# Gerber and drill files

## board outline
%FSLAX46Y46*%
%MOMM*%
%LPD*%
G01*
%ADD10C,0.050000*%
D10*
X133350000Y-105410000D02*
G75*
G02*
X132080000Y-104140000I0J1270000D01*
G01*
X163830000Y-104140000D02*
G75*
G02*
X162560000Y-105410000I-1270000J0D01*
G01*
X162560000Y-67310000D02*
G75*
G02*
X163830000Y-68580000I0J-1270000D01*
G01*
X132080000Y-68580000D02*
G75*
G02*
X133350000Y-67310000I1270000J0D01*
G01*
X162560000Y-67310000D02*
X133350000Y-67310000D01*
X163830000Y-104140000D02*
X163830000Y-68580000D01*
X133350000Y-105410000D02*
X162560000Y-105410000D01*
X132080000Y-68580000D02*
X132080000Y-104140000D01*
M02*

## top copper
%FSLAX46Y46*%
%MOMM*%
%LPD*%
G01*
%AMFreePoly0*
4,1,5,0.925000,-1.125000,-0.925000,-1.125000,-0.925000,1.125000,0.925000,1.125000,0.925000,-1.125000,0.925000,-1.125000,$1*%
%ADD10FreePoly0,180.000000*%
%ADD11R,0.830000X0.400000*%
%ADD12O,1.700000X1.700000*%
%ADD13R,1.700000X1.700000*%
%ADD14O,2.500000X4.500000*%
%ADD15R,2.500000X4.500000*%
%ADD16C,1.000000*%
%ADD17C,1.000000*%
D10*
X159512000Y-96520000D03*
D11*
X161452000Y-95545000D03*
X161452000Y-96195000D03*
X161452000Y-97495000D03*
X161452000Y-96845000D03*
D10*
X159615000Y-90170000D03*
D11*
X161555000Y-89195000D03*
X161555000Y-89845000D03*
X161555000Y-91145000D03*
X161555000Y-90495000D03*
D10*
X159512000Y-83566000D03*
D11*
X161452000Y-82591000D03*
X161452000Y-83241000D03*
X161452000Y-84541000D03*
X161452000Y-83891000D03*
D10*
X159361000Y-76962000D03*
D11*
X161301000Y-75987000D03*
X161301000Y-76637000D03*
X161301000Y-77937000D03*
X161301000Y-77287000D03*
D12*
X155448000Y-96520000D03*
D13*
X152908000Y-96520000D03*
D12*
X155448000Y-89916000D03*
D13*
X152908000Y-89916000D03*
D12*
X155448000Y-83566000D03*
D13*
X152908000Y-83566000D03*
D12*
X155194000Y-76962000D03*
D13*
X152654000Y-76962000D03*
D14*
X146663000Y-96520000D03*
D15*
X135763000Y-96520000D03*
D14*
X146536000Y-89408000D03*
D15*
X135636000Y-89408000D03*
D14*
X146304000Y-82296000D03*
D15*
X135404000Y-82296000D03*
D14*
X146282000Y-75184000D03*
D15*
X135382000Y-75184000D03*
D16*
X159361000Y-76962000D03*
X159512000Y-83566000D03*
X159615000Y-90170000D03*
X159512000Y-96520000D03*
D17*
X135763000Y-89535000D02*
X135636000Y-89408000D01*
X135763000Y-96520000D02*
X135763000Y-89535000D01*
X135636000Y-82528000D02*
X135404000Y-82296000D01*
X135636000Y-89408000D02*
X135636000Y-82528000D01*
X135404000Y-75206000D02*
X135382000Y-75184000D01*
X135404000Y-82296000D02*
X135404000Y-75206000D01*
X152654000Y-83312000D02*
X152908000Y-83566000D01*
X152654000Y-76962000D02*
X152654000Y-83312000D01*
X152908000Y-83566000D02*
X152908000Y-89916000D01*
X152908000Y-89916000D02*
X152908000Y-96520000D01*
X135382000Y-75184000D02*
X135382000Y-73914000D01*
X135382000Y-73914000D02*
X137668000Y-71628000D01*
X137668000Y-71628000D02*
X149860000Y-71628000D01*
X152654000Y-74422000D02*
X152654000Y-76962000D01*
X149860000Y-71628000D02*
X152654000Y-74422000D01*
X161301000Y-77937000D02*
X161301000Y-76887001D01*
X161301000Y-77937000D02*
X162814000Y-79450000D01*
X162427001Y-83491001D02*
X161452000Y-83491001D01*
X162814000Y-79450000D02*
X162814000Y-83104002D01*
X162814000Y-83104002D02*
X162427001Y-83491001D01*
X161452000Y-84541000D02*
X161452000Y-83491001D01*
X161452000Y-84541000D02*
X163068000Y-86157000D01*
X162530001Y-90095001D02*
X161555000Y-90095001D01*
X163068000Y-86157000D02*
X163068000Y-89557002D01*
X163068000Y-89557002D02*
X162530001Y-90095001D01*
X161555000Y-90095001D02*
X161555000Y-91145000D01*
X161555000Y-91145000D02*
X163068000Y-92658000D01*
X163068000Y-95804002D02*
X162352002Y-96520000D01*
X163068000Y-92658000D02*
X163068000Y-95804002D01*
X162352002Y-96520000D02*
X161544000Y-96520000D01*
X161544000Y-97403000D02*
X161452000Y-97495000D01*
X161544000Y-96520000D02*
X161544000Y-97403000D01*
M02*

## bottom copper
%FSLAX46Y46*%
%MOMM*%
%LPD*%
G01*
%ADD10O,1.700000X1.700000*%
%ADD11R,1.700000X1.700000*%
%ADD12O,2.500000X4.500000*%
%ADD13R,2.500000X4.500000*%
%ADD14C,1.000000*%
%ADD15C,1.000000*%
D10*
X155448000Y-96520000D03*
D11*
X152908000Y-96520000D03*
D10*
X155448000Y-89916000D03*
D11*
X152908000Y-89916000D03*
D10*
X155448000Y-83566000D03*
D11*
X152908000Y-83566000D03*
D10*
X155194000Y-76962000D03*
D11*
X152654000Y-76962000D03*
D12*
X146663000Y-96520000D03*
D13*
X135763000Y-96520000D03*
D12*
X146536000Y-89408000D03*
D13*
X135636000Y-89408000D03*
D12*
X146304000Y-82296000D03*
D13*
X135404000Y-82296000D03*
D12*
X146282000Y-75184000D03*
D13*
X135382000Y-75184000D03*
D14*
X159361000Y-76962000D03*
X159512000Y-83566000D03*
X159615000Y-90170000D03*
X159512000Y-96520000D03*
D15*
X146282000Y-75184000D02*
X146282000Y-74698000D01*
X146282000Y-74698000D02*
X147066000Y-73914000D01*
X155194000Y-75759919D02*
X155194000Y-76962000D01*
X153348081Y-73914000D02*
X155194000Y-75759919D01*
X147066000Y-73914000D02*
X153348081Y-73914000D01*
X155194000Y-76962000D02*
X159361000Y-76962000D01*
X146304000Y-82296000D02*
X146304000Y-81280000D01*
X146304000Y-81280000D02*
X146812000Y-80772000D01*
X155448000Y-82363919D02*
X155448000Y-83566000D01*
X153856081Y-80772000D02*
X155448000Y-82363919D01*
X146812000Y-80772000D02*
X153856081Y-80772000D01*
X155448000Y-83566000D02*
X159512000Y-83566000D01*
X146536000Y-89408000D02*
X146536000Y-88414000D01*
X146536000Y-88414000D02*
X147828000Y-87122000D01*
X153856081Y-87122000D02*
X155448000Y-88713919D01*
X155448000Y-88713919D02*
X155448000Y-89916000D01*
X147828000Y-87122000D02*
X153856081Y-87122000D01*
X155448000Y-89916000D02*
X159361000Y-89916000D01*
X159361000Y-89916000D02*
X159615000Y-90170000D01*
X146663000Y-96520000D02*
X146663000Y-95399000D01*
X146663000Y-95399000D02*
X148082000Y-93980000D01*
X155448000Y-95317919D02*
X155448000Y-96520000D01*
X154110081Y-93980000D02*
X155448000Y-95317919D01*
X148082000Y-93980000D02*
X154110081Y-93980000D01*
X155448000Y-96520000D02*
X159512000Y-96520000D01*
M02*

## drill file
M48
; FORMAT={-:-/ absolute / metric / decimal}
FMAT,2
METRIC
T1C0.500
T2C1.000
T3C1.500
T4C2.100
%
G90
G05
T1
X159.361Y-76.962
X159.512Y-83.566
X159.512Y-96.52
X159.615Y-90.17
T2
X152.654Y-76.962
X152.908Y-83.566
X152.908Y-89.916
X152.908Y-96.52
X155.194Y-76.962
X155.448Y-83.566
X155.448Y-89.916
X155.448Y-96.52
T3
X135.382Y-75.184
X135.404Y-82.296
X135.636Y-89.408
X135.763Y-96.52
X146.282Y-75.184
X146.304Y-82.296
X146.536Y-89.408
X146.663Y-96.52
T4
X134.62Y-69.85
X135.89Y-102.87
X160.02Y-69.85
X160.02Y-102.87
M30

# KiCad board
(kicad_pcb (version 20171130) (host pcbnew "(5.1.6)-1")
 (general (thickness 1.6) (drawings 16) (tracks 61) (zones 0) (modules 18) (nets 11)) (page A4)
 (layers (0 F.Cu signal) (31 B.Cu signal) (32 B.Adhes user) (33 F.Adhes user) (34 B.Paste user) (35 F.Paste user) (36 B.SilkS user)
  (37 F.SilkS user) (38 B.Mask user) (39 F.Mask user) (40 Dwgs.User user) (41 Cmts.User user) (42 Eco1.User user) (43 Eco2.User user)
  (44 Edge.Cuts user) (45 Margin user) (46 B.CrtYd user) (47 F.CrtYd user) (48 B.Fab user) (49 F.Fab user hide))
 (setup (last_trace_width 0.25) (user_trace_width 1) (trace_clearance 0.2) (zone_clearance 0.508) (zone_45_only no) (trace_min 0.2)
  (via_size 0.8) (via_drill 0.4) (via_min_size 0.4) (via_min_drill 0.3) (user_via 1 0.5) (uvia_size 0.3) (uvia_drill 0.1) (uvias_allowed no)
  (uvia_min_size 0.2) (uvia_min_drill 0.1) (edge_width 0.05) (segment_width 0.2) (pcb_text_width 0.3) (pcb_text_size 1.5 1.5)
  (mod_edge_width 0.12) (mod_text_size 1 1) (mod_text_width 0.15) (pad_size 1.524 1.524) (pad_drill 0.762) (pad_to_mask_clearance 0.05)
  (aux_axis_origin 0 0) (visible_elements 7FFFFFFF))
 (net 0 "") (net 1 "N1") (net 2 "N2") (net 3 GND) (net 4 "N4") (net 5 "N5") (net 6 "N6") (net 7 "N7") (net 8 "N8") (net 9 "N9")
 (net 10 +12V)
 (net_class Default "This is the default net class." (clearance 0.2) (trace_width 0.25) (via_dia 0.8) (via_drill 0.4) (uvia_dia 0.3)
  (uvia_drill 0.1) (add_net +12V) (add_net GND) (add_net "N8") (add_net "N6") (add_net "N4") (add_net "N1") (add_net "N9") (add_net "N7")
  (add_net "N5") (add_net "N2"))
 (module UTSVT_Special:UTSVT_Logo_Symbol (layer B.Cu) (at 137.16 91.44 90)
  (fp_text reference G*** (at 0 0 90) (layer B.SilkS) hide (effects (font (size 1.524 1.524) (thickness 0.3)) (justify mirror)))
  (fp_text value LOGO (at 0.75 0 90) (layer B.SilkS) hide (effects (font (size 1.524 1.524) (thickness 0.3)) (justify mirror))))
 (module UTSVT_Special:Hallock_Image (layer B.Cu) (at 146.685 89.535)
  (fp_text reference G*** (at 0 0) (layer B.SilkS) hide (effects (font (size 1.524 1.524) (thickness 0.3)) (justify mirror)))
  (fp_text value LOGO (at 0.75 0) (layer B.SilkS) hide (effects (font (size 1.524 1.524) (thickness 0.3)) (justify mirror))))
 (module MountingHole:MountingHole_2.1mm (layer F.Cu) (at 134.62 69.85)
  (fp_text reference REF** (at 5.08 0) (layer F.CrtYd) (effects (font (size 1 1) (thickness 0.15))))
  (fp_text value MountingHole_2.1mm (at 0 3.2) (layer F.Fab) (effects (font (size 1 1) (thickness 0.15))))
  (pad "" np_thru_hole circle (at 0 0) (size 2.1 2.1) (drill 2.1) (layers *.Cu *.Mask)))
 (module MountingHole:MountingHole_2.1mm (layer F.Cu) (at 135.89 102.87)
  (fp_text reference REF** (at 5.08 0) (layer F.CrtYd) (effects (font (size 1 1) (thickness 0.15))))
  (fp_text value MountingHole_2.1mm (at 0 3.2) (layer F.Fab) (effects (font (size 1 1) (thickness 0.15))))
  (pad "" np_thru_hole circle (at 0 0) (size 2.1 2.1) (drill 2.1) (layers *.Cu *.Mask)))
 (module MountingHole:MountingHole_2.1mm (layer F.Cu) (at 160.02 102.87)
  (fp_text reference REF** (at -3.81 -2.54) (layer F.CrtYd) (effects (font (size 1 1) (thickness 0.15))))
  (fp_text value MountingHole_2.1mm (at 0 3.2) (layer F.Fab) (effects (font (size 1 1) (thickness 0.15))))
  (pad "" np_thru_hole circle (at 0 0) (size 2.1 2.1) (drill 2.1) (layers *.Cu *.Mask)))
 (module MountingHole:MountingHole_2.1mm (layer F.Cu) (at 160.02 69.85)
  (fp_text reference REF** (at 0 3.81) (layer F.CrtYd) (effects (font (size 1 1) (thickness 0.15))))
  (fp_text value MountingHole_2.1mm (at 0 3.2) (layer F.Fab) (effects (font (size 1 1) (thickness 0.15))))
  (pad "" np_thru_hole circle (at 0 0) (size 2.1 2.1) (drill 2.1) (layers *.Cu *.Mask)))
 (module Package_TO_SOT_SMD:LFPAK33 (layer F.Cu) (at 159.917 96.52 180) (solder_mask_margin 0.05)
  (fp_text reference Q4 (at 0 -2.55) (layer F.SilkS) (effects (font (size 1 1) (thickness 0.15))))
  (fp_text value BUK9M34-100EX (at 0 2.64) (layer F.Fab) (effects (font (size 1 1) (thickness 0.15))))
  (pad 5 smd custom (at 0.405 0 180) (size 1.85 2.25) (layers F.Cu F.Mask) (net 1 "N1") (zone_connect 2)
   (options (clearance outline) (anchor rect)) (primitives))
  (pad "" smd rect (at 1.575 0.975 180) (size 0.75 0.3) (layers F.Paste))
  (pad "" smd rect (at 1.575 0.325 180) (size 0.75 0.3) (layers F.Paste))
  (pad "" smd rect (at 1.575 -0.325 180) (size 0.75 0.3) (layers F.Paste))
  (pad "" smd rect (at 1.575 -0.975 180) (size 0.75 0.3) (layers F.Paste))
  (pad "" smd rect (at -1.535 -0.975 180) (size 0.83 0.3) (layers F.Paste))
  (pad "" smd rect (at -1.535 -0.325 180) (size 0.83 0.3) (layers F.Paste))
  (pad "" smd rect (at -1.535 0.325 180) (size 0.83 0.3) (layers F.Paste))
  (pad 4 smd rect (at -1.535 0.975 180) (size 0.83 0.4) (layers F.Cu F.Mask) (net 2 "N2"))
  (pad "" smd rect (at -1.535 0.975 180) (size 0.83 0.3) (layers F.Paste))
  (pad 3 smd rect (at -1.535 0.325 180) (size 0.83 0.4) (layers F.Cu F.Mask) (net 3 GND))
  (pad 1 smd rect (at -1.535 -0.975 180) (size 0.83 0.4) (layers F.Cu F.Mask) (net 3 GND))
  (pad 2 smd rect (at -1.535 -0.325 180) (size 0.83 0.4) (layers F.Cu F.Mask) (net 3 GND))
  (pad "" smd rect (at 0.645 0.626 180) (size 0.51 0.635) (layers F.Paste))
  (pad "" smd rect (at -0.215 0.626 180) (size 0.51 0.635) (layers F.Paste))
  (pad "" smd rect (at 0.645 -0.626 180) (size 0.51 0.635) (layers F.Paste))
  (pad "" smd rect (at -0.215 -0.626 180) (size 0.51 0.635) (layers F.Paste)))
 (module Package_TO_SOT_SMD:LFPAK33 (layer F.Cu) (at 160.02 90.17 180) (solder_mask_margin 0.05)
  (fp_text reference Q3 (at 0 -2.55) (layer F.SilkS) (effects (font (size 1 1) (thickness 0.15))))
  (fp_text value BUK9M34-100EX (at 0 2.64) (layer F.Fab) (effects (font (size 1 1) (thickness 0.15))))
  (pad 5 smd custom (at 0.405 0 180) (size 1.85 2.25) (layers F.Cu F.Mask) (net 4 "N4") (zone_connect 2)
   (options (clearance outline) (anchor rect)) (primitives))
  (pad "" smd rect (at 1.575 0.975 180) (size 0.75 0.3) (layers F.Paste))
  (pad "" smd rect (at 1.575 0.325 180) (size 0.75 0.3) (layers F.Paste))
  (pad "" smd rect (at 1.575 -0.325 180) (size 0.75 0.3) (layers F.Paste))
  (pad "" smd rect (at 1.575 -0.975 180) (size 0.75 0.3) (layers F.Paste))
  (pad "" smd rect (at -1.535 -0.975 180) (size 0.83 0.3) (layers F.Paste))
  (pad "" smd rect (at -1.535 -0.325 180) (size 0.83 0.3) (layers F.Paste))
  (pad "" smd rect (at -1.535 0.325 180) (size 0.83 0.3) (layers F.Paste))
  (pad 4 smd rect (at -1.535 0.975 180) (size 0.83 0.4) (layers F.Cu F.Mask) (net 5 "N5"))
  (pad "" smd rect (at -1.535 0.975 180) (size 0.83 0.3) (layers F.Paste))
  (pad 3 smd rect (at -1.535 0.325 180) (size 0.83 0.4) (layers F.Cu F.Mask) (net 3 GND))
  (pad 1 smd rect (at -1.535 -0.975 180) (size 0.83 0.4) (layers F.Cu F.Mask) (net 3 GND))
  (pad 2 smd rect (at -1.535 -0.325 180) (size 0.83 0.4) (layers F.Cu F.Mask) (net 3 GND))
  (pad "" smd rect (at 0.645 0.626 180) (size 0.51 0.635) (layers F.Paste))
  (pad "" smd rect (at -0.215 0.626 180) (size 0.51 0.635) (layers F.Paste))
  (pad "" smd rect (at 0.645 -0.626 180) (size 0.51 0.635) (layers F.Paste))
  (pad "" smd rect (at -0.215 -0.626 180) (size 0.51 0.635) (layers F.Paste)))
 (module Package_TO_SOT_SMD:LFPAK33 (layer F.Cu) (at 159.917 83.566 180) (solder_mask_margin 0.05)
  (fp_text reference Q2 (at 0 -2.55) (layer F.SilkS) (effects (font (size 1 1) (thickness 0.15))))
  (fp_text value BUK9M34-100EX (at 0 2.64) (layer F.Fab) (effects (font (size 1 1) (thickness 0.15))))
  (pad 5 smd custom (at 0.405 0 180) (size 1.85 2.25) (layers F.Cu F.Mask) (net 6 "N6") (zone_connect 2)
   (options (clearance outline) (anchor rect)) (primitives))
  (pad "" smd rect (at 1.575 0.975 180) (size 0.75 0.3) (layers F.Paste))
  (pad "" smd rect (at 1.575 0.325 180) (size 0.75 0.3) (layers F.Paste))
  (pad "" smd rect (at 1.575 -0.325 180) (size 0.75 0.3) (layers F.Paste))
  (pad "" smd rect (at 1.575 -0.975 180) (size 0.75 0.3) (layers F.Paste))
  (pad "" smd rect (at -1.535 -0.975 180) (size 0.83 0.3) (layers F.Paste))
  (pad "" smd rect (at -1.535 -0.325 180) (size 0.83 0.3) (layers F.Paste))
  (pad "" smd rect (at -1.535 0.325 180) (size 0.83 0.3) (layers F.Paste))
  (pad 4 smd rect (at -1.535 0.975 180) (size 0.83 0.4) (layers F.Cu F.Mask) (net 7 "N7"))
  (pad "" smd rect (at -1.535 0.975 180) (size 0.83 0.3) (layers F.Paste))
  (pad 3 smd rect (at -1.535 0.325 180) (size 0.83 0.4) (layers F.Cu F.Mask) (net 3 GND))
  (pad 1 smd rect (at -1.535 -0.975 180) (size 0.83 0.4) (layers F.Cu F.Mask) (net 3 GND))
  (pad 2 smd rect (at -1.535 -0.325 180) (size 0.83 0.4) (layers F.Cu F.Mask) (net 3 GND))
  (pad "" smd rect (at 0.645 0.626 180) (size 0.51 0.635) (layers F.Paste))
  (pad "" smd rect (at -0.215 0.626 180) (size 0.51 0.635) (layers F.Paste))
  (pad "" smd rect (at 0.645 -0.626 180) (size 0.51 0.635) (layers F.Paste))
  (pad "" smd rect (at -0.215 -0.626 180) (size 0.51 0.635) (layers F.Paste)))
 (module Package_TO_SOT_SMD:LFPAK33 (layer F.Cu) (at 159.766 76.962 180) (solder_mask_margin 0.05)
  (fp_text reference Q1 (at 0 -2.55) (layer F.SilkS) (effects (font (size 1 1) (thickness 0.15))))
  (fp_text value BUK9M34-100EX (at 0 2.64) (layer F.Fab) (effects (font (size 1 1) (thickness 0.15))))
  (pad 5 smd custom (at 0.405 0 180) (size 1.85 2.25) (layers F.Cu F.Mask) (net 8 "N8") (zone_connect 2)
   (options (clearance outline) (anchor rect)) (primitives))
  (pad "" smd rect (at 1.575 0.975 180) (size 0.75 0.3) (layers F.Paste))
  (pad "" smd rect (at 1.575 0.325 180) (size 0.75 0.3) (layers F.Paste))
  (pad "" smd rect (at 1.575 -0.325 180) (size 0.75 0.3) (layers F.Paste))
  (pad "" smd rect (at 1.575 -0.975 180) (size 0.75 0.3) (layers F.Paste))
  (pad "" smd rect (at -1.535 -0.975 180) (size 0.83 0.3) (layers F.Paste))
  (pad "" smd rect (at -1.535 -0.325 180) (size 0.83 0.3) (layers F.Paste))
  (pad "" smd rect (at -1.535 0.325 180) (size 0.83 0.3) (layers F.Paste))
  (pad 4 smd rect (at -1.535 0.975 180) (size 0.83 0.4) (layers F.Cu F.Mask) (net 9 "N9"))
  (pad "" smd rect (at -1.535 0.975 180) (size 0.83 0.3) (layers F.Paste))
  (pad 3 smd rect (at -1.535 0.325 180) (size 0.83 0.4) (layers F.Cu F.Mask) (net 3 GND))
  (pad 1 smd rect (at -1.535 -0.975 180) (size 0.83 0.4) (layers F.Cu F.Mask) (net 3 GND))
  (pad 2 smd rect (at -1.535 -0.325 180) (size 0.83 0.4) (layers F.Cu F.Mask) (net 3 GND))
  (pad "" smd rect (at 0.645 0.626 180) (size 0.51 0.635) (layers F.Paste))
  (pad "" smd rect (at -0.215 0.626 180) (size 0.51 0.635) (layers F.Paste))
  (pad "" smd rect (at 0.645 -0.626 180) (size 0.51 0.635) (layers F.Paste))
  (pad "" smd rect (at -0.215 -0.626 180) (size 0.51 0.635) (layers F.Paste)))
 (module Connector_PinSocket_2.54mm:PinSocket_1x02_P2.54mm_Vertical (layer F.Cu) (at 152.908 96.52 90)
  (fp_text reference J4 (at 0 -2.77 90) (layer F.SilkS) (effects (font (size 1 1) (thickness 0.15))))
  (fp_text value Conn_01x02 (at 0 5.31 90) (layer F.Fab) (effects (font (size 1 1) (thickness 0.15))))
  (pad 2 thru_hole oval (at 0 2.54 90) (size 1.7 1.7) (drill 1) (layers *.Cu *.Mask) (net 1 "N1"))
  (pad 1 thru_hole rect (at 0 0 90) (size 1.7 1.7) (drill 1) (layers *.Cu *.Mask) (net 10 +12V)))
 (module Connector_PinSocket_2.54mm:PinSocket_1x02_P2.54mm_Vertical (layer F.Cu) (at 152.908 89.916 90)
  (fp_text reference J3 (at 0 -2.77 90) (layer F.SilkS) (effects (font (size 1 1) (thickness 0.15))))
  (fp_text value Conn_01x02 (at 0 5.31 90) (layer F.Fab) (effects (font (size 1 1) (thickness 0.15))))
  (pad 2 thru_hole oval (at 0 2.54 90) (size 1.7 1.7) (drill 1) (layers *.Cu *.Mask) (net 4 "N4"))
  (pad 1 thru_hole rect (at 0 0 90) (size 1.7 1.7) (drill 1) (layers *.Cu *.Mask) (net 10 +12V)))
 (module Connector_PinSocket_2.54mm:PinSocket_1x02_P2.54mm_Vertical (layer F.Cu) (at 152.908 83.566 90)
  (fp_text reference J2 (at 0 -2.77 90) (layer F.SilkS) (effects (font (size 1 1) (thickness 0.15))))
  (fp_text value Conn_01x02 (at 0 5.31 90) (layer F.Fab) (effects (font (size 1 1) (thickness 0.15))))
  (pad 2 thru_hole oval (at 0 2.54 90) (size 1.7 1.7) (drill 1) (layers *.Cu *.Mask) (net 6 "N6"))
  (pad 1 thru_hole rect (at 0 0 90) (size 1.7 1.7) (drill 1) (layers *.Cu *.Mask) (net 10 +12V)))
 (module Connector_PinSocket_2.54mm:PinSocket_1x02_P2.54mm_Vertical (layer F.Cu) (at 152.654 76.962 90)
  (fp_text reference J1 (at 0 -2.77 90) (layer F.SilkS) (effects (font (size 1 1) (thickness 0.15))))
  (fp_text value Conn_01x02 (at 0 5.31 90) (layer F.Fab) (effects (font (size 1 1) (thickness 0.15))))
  (pad 2 thru_hole oval (at 0 2.54 90) (size 1.7 1.7) (drill 1) (layers *.Cu *.Mask) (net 8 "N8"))
  (pad 1 thru_hole rect (at 0 0 90) (size 1.7 1.7) (drill 1) (layers *.Cu *.Mask) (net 10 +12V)))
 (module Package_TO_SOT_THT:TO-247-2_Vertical (layer F.Cu) (at 135.763 96.52)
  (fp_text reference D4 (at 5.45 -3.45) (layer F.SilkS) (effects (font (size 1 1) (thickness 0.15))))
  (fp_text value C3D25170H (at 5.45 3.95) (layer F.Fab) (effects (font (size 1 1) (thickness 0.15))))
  (pad 2 thru_hole oval (at 10.9 0) (size 2.5 4.5) (drill 1.5) (layers *.Cu *.Mask) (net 1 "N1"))
  (pad 1 thru_hole rect (at 0 0) (size 2.5 4.5) (drill 1.5) (layers *.Cu *.Mask) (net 10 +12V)))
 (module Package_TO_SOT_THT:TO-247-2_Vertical (layer F.Cu) (at 135.636 89.408)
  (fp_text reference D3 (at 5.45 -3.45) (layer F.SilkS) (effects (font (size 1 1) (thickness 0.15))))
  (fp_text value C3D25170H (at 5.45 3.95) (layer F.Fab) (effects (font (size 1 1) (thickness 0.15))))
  (pad 2 thru_hole oval (at 10.9 0) (size 2.5 4.5) (drill 1.5) (layers *.Cu *.Mask) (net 4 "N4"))
  (pad 1 thru_hole rect (at 0 0) (size 2.5 4.5) (drill 1.5) (layers *.Cu *.Mask) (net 10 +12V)))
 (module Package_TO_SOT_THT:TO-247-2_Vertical (layer F.Cu) (at 135.404 82.296)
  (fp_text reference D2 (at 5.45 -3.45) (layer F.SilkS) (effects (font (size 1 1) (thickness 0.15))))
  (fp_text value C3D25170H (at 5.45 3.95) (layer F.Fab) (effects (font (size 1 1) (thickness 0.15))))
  (pad 2 thru_hole oval (at 10.9 0) (size 2.5 4.5) (drill 1.5) (layers *.Cu *.Mask) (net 6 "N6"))
  (pad 1 thru_hole rect (at 0 0) (size 2.5 4.5) (drill 1.5) (layers *.Cu *.Mask) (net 10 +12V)))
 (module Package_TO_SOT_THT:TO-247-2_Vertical (layer F.Cu) (at 135.382 75.184)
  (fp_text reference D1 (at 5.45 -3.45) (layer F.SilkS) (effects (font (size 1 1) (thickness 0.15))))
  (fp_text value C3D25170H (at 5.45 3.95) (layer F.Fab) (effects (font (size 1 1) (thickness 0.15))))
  (pad 2 thru_hole oval (at 10.9 0) (size 2.5 4.5) (drill 1.5) (layers *.Cu *.Mask) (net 8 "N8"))
  (pad 1 thru_hole rect (at 0 0) (size 2.5 4.5) (drill 1.5) (layers *.Cu *.Mask) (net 10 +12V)))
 (gr_arc (start 133.35 104.14) (end 132.08 104.14) (angle -90) (layer Edge.Cuts) (width 0.05))
 (gr_arc (start 162.56 104.14) (end 162.56 105.41) (angle -90) (layer Edge.Cuts) (width 0.05))
 (gr_arc (start 162.56 68.58) (end 163.83 68.58) (angle -90) (layer Edge.Cuts) (width 0.05))
 (gr_arc (start 133.35 68.58) (end 133.35 67.31) (angle -90) (layer Edge.Cuts) (width 0.05))
 (gr_line (start 162.56 67.31) (end 133.35 67.31) (layer Edge.Cuts) (width 0.05))
 (gr_line (start 163.83 104.14) (end 163.83 68.58) (layer Edge.Cuts) (width 0.05))
 (gr_line (start 133.35 105.41) (end 162.56 105.41) (layer Edge.Cuts) (width 0.05))
 (gr_line (start 132.08 68.58) (end 132.08 104.14) (layer Edge.Cuts) (width 0.05))
 (segment (start 146.282 75.184) (end 146.282 74.698) (width 1) (layer B.Cu) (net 8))
 (segment (start 146.282 74.698) (end 147.066 73.914) (width 1) (layer B.Cu) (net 8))
 (segment (start 155.194 75.759919) (end 155.194 76.962) (width 1) (layer B.Cu) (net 8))
 (segment (start 153.348081 73.914) (end 155.194 75.759919) (width 1) (layer B.Cu) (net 8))
 (segment (start 147.066 73.914) (end 153.348081 73.914) (width 1) (layer B.Cu) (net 8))
 (segment (start 155.194 76.962) (end 159.361 76.962) (width 1) (layer B.Cu) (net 8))
 (via (at 159.361 76.962) (size 1) (drill 0.5) (layers F.Cu B.Cu) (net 8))
 (segment (start 135.763 89.535) (end 135.636 89.408) (width 1) (layer F.Cu) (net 10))
 (segment (start 135.763 96.52) (end 135.763 89.535) (width 1) (layer F.Cu) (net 10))
 (segment (start 135.636 82.528) (end 135.404 82.296) (width 1) (layer F.Cu) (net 10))
 (segment (start 135.636 89.408) (end 135.636 82.528) (width 1) (layer F.Cu) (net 10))
 (segment (start 135.404 75.206) (end 135.382 75.184) (width 1) (layer F.Cu) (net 10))
 (segment (start 135.404 82.296) (end 135.404 75.206) (width 1) (layer F.Cu) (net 10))
 (segment (start 152.654 83.312) (end 152.908 83.566) (width 1) (layer F.Cu) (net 10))
 (segment (start 152.654 76.962) (end 152.654 83.312) (width 1) (layer F.Cu) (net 10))
 (segment (start 152.908 83.566) (end 152.908 89.916) (width 1) (layer F.Cu) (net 10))
 (segment (start 152.908 89.916) (end 152.908 96.52) (width 1) (layer F.Cu) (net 10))
 (segment (start 135.382 75.184) (end 135.382 73.914) (width 1) (layer F.Cu) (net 10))
 (segment (start 135.382 73.914) (end 137.668 71.628) (width 1) (layer F.Cu) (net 10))
 (segment (start 137.668 71.628) (end 149.86 71.628) (width 1) (layer F.Cu) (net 10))
 (segment (start 152.654 74.422) (end 152.654 76.962) (width 1) (layer F.Cu) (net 10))
 (segment (start 149.86 71.628) (end 152.654 74.422) (width 1) (layer F.Cu) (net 10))
 (segment (start 146.304 82.296) (end 146.304 81.28) (width 1) (layer B.Cu) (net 6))
 (segment (start 146.304 81.28) (end 146.812 80.772) (width 1) (layer B.Cu) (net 6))
 (segment (start 155.448 82.363919) (end 155.448 83.566) (width 1) (layer B.Cu) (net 6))
 (segment (start 153.856081 80.772) (end 155.448 82.363919) (width 1) (layer B.Cu) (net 6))
 (segment (start 146.812 80.772) (end 153.856081 80.772) (width 1) (layer B.Cu) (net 6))
 (via (at 159.512 83.566) (size 1) (drill 0.5) (layers F.Cu B.Cu) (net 6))
 (segment (start 155.448 83.566) (end 159.512 83.566) (width 1) (layer B.Cu) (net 6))
 (segment (start 146.536 89.408) (end 146.536 88.414) (width 1) (layer B.Cu) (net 4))
 (segment (start 146.536 88.414) (end 147.828 87.122) (width 1) (layer B.Cu) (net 4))
 (segment (start 153.856081 87.122) (end 155.448 88.713919) (width 1) (layer B.Cu) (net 4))
 (segment (start 155.448 88.713919) (end 155.448 89.916) (width 1) (layer B.Cu) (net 4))
 (segment (start 147.828 87.122) (end 153.856081 87.122) (width 1) (layer B.Cu) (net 4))
 (via (at 159.615 90.17) (size 1) (drill 0.5) (layers F.Cu B.Cu) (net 4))
 (segment (start 155.448 89.916) (end 159.361 89.916) (width 1) (layer B.Cu) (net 4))
 (segment (start 159.361 89.916) (end 159.615 90.17) (width 1) (layer B.Cu) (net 4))
 (segment (start 146.663 96.52) (end 146.663 95.399) (width 1) (layer B.Cu) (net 1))
 (segment (start 146.663 95.399) (end 148.082 93.98) (width 1) (layer B.Cu) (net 1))
 (segment (start 155.448 95.317919) (end 155.448 96.52) (width 1) (layer B.Cu) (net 1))
 (segment (start 154.110081 93.98) (end 155.448 95.317919) (width 1) (layer B.Cu) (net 1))
 (segment (start 148.082 93.98) (end 154.110081 93.98) (width 1) (layer B.Cu) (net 1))
 (via (at 159.512 96.52) (size 1) (drill 0.5) (layers F.Cu B.Cu) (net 1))
 (segment (start 155.448 96.52) (end 159.512 96.52) (width 1) (layer B.Cu) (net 1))
 (segment (start 161.301 77.937) (end 161.301 76.887001) (width 1) (layer F.Cu) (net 3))
 (segment (start 161.301 77.937) (end 162.814 79.45) (width 1) (layer F.Cu) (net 3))
 (segment (start 162.427001 83.491001) (end 161.452 83.491001) (width 1) (layer F.Cu) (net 3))
 (segment (start 162.814 79.45) (end 162.814 83.104002) (width 1) (layer F.Cu) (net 3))
 (segment (start 162.814 83.104002) (end 162.427001 83.491001) (width 1) (layer F.Cu) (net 3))
 (segment (start 161.452 84.541) (end 161.452 83.491001) (width 1) (layer F.Cu) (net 3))
 (segment (start 161.452 84.541) (end 163.068 86.157) (width 1) (layer F.Cu) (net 3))
 (segment (start 162.530001 90.095001) (end 161.555 90.095001) (width 1) (layer F.Cu) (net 3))
 (segment (start 163.068 86.157) (end 163.068 89.557002) (width 1) (layer F.Cu) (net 3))
 (segment (start 163.068 89.557002) (end 162.530001 90.095001) (width 1) (layer F.Cu) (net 3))
 (segment (start 161.555 90.095001) (end 161.555 91.145) (width 1) (layer F.Cu) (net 3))
 (segment (start 161.555 91.145) (end 163.068 92.658) (width 1) (layer F.Cu) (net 3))
 (segment (start 163.068 95.804002) (end 162.352002 96.52) (width 1) (layer F.Cu) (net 3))
 (segment (start 163.068 92.658) (end 163.068 95.804002) (width 1) (layer F.Cu) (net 3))
 (segment (start 162.352002 96.52) (end 161.544 96.52) (width 1) (layer F.Cu) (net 3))
 (segment (start 161.544 97.403) (end 161.452 97.495) (width 1) (layer F.Cu) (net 3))
 (segment (start 161.544 96.52) (end 161.544 97.403) (width 1) (layer F.Cu) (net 3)))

